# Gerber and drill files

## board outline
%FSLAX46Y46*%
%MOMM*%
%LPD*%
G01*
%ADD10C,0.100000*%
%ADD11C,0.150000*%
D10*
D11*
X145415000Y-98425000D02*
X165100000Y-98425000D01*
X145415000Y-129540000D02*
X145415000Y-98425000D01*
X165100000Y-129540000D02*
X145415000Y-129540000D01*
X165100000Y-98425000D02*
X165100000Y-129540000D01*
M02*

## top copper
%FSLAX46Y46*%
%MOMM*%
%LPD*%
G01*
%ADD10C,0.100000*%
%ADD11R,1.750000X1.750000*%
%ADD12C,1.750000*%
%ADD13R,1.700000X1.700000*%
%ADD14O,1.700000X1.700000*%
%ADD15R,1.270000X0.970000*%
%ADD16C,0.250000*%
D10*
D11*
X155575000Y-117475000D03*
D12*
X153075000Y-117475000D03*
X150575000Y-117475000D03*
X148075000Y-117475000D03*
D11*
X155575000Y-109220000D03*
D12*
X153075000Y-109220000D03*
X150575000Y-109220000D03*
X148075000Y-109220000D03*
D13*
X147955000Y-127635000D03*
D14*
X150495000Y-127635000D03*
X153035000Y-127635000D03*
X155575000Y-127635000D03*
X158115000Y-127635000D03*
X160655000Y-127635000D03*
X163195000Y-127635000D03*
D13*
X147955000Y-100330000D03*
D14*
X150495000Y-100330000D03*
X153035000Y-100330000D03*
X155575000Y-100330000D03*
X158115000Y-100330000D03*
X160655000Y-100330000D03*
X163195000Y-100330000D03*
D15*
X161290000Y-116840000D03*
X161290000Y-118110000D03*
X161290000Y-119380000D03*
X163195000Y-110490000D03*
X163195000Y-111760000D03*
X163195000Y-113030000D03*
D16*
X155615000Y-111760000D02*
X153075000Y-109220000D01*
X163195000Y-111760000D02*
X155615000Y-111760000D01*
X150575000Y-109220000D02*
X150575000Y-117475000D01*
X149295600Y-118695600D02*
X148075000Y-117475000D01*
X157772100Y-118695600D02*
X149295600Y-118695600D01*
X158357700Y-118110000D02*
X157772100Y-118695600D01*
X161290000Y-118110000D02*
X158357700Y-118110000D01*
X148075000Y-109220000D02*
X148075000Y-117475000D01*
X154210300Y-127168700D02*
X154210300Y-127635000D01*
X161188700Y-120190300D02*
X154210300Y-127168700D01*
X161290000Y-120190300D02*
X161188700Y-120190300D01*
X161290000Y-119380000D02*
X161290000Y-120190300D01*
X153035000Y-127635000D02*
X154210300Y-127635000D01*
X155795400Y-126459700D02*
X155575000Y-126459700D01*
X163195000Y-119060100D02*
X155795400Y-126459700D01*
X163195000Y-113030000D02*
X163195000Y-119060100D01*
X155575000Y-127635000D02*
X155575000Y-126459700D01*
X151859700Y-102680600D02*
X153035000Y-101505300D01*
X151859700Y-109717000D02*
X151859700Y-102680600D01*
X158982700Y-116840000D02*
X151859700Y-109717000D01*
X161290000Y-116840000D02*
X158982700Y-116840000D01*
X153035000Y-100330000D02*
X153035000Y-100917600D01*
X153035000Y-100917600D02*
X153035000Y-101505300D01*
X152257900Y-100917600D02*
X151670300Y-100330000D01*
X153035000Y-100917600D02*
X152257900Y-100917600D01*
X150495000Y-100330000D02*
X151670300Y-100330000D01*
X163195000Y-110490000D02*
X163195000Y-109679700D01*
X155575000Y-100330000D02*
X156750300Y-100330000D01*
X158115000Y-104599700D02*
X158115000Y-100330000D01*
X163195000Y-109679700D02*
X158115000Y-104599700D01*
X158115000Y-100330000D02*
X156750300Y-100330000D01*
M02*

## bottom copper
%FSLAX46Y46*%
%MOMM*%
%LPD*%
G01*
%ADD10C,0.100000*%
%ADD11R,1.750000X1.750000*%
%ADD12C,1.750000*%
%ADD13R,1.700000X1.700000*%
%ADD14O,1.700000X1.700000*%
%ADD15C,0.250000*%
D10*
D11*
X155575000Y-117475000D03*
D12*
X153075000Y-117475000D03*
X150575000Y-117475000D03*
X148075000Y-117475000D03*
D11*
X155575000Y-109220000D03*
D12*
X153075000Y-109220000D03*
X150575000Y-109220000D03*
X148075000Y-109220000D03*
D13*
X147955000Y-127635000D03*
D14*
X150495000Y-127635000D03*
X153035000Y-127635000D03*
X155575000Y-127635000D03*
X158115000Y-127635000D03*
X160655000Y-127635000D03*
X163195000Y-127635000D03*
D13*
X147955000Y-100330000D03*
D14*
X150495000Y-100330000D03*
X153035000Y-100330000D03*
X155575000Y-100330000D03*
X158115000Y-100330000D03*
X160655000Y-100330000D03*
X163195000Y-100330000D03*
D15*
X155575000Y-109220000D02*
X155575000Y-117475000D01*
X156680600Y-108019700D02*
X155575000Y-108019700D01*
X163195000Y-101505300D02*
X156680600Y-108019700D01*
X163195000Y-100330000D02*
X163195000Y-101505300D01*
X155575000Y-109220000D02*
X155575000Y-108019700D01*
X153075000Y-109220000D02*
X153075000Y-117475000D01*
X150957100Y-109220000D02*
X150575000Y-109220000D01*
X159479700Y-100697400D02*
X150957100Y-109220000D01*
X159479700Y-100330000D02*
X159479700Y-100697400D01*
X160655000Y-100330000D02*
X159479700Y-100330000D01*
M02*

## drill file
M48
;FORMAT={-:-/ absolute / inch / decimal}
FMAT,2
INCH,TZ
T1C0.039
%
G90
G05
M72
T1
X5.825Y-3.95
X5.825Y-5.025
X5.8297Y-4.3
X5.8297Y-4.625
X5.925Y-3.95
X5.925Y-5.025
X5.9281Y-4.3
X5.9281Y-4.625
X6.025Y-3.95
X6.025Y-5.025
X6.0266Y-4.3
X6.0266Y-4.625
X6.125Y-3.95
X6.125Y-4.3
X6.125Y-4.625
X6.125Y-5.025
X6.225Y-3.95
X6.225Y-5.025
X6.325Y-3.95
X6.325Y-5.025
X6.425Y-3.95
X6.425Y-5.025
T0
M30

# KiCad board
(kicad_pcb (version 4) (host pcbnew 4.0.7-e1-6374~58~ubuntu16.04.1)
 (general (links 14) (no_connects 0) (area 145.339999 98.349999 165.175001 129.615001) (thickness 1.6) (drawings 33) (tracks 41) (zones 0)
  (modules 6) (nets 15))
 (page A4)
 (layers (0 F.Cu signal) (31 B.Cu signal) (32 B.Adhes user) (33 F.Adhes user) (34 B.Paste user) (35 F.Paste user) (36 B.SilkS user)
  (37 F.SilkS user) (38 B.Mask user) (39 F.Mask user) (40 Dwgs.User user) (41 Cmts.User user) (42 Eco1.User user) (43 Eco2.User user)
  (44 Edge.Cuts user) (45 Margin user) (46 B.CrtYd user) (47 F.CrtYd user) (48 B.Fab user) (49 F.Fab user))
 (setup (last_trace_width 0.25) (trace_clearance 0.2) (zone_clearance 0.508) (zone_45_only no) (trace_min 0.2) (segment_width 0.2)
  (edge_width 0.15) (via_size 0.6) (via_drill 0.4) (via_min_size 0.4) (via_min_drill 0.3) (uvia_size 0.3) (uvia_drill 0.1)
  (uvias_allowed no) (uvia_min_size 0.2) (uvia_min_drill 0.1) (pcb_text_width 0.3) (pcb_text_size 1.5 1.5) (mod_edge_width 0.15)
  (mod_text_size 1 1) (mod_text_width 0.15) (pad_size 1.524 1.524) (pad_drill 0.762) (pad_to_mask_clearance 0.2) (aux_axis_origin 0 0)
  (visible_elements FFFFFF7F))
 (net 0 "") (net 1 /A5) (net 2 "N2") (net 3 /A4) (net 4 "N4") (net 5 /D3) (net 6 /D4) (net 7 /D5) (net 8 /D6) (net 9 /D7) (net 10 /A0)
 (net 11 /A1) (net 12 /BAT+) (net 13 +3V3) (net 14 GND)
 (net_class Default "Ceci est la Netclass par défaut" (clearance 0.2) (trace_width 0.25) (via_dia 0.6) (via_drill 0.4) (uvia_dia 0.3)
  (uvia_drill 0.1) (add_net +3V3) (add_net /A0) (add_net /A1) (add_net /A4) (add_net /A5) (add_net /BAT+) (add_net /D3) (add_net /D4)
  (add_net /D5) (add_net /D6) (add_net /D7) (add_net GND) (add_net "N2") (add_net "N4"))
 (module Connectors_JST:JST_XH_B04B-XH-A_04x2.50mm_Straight (layer F.Cu) (at 155.575 117.475 180)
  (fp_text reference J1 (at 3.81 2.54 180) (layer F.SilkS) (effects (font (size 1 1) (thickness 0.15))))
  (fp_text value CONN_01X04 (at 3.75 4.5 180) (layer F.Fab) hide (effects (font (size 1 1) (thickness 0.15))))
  (pad 1 thru_hole rect (at 0 0 180) (size 1.75 1.75) (drill 1) (layers *.Cu *.Mask) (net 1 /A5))
  (pad 2 thru_hole circle (at 2.5 0 180) (size 1.75 1.75) (drill 1) (layers *.Cu *.Mask) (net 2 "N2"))
  (pad 3 thru_hole circle (at 5 0 180) (size 1.75 1.75) (drill 1) (layers *.Cu *.Mask) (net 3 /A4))
  (pad 4 thru_hole circle (at 7.5 0 180) (size 1.75 1.75) (drill 1) (layers *.Cu *.Mask) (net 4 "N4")))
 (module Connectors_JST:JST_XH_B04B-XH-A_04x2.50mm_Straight (layer F.Cu) (at 155.575 109.22 180)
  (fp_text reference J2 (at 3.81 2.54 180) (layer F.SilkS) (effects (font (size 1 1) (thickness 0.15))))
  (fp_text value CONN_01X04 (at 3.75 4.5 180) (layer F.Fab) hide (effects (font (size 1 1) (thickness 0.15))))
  (pad 1 thru_hole rect (at 0 0 180) (size 1.75 1.75) (drill 1) (layers *.Cu *.Mask) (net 1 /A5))
  (pad 2 thru_hole circle (at 2.5 0 180) (size 1.75 1.75) (drill 1) (layers *.Cu *.Mask) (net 2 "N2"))
  (pad 3 thru_hole circle (at 5 0 180) (size 1.75 1.75) (drill 1) (layers *.Cu *.Mask) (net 3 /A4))
  (pad 4 thru_hole circle (at 7.5 0 180) (size 1.75 1.75) (drill 1) (layers *.Cu *.Mask) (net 4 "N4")))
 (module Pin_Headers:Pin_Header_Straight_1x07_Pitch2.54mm (layer B.Cu) (at 147.955 127.635 270)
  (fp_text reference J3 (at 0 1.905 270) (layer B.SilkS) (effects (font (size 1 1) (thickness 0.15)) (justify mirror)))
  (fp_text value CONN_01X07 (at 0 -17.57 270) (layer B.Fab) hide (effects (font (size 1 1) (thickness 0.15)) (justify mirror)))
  (pad 1 thru_hole rect (at 0 0 270) (size 1.7 1.7) (drill 1) (layers *.Cu *.Mask) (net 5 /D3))
  (pad 2 thru_hole oval (at 0 -2.54 270) (size 1.7 1.7) (drill 1) (layers *.Cu *.Mask) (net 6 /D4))
  (pad 3 thru_hole oval (at 0 -5.08 270) (size 1.7 1.7) (drill 1) (layers *.Cu *.Mask) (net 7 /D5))
  (pad 4 thru_hole oval (at 0 -7.62 270) (size 1.7 1.7) (drill 1) (layers *.Cu *.Mask) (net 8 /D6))
  (pad 5 thru_hole oval (at 0 -10.16 270) (size 1.7 1.7) (drill 1) (layers *.Cu *.Mask) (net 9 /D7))
  (pad 6 thru_hole oval (at 0 -12.7 270) (size 1.7 1.7) (drill 1) (layers *.Cu *.Mask) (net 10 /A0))
  (pad 7 thru_hole oval (at 0 -15.24 270) (size 1.7 1.7) (drill 1) (layers *.Cu *.Mask) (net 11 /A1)))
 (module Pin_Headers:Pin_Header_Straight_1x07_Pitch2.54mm (layer B.Cu) (at 147.955 100.33 270)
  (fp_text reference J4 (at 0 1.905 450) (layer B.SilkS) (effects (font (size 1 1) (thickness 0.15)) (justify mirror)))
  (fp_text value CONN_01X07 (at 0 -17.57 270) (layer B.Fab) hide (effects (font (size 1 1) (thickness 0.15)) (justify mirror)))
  (pad 1 thru_hole rect (at 0 0 270) (size 1.7 1.7) (drill 1) (layers *.Cu *.Mask) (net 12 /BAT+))
  (pad 2 thru_hole oval (at 0 -2.54 270) (size 1.7 1.7) (drill 1) (layers *.Cu *.Mask) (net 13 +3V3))
  (pad 3 thru_hole oval (at 0 -5.08 270) (size 1.7 1.7) (drill 1) (layers *.Cu *.Mask) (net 13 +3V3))
  (pad 4 thru_hole oval (at 0 -7.62 270) (size 1.7 1.7) (drill 1) (layers *.Cu *.Mask) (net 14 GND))
  (pad 5 thru_hole oval (at 0 -10.16 270) (size 1.7 1.7) (drill 1) (layers *.Cu *.Mask) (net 14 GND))
  (pad 6 thru_hole oval (at 0 -12.7 270) (size 1.7 1.7) (drill 1) (layers *.Cu *.Mask) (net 3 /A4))
  (pad 7 thru_hole oval (at 0 -15.24 270) (size 1.7 1.7) (drill 1) (layers *.Cu *.Mask) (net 1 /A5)))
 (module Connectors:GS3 (layer F.Cu) (at 161.29 118.11)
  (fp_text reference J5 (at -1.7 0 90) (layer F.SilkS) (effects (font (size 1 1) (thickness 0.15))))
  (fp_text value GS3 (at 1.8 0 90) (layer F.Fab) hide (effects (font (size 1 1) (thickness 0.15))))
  (pad 1 smd rect (at 0 -1.27) (size 1.27 0.97) (layers F.Cu F.Paste F.Mask) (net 13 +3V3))
  (pad 2 smd rect (at 0 0) (size 1.27 0.97) (layers F.Cu F.Paste F.Mask) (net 4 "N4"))
  (pad 3 smd rect (at 0 1.27) (size 1.27 0.97) (layers F.Cu F.Paste F.Mask) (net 7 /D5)))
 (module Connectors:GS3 (layer F.Cu) (at 163.195 111.76)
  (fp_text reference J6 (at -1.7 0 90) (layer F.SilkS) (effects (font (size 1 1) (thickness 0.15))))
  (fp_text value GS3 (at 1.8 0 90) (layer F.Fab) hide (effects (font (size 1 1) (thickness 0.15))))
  (pad 1 smd rect (at 0 -1.27) (size 1.27 0.97) (layers F.Cu F.Paste F.Mask) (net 14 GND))
  (pad 2 smd rect (at 0 0) (size 1.27 0.97) (layers F.Cu F.Paste F.Mask) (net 2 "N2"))
  (pad 3 smd rect (at 0 1.27) (size 1.27 0.97) (layers F.Cu F.Paste F.Mask) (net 8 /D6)))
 (gr_line (start 145.415 98.425) (end 165.1 98.425) (angle 90) (layer Edge.Cuts) (width 0.15))
 (gr_line (start 145.415 129.54) (end 145.415 98.425) (angle 90) (layer Edge.Cuts) (width 0.15))
 (gr_line (start 165.1 129.54) (end 145.415 129.54) (angle 90) (layer Edge.Cuts) (width 0.15))
 (gr_line (start 165.1 98.425) (end 165.1 129.54) (angle 90) (layer Edge.Cuts) (width 0.15))
 (segment (start 155.575 109.22) (end 155.575 117.475) (width 0.25) (layer B.Cu) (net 1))
 (segment (start 156.6806 108.0197) (end 155.575 108.0197) (width 0.25) (layer B.Cu) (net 1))
 (segment (start 163.195 101.5053) (end 156.6806 108.0197) (width 0.25) (layer B.Cu) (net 1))
 (segment (start 163.195 100.33) (end 163.195 101.5053) (width 0.25) (layer B.Cu) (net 1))
 (segment (start 155.575 109.22) (end 155.575 108.0197) (width 0.25) (layer B.Cu) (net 1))
 (segment (start 155.615 111.76) (end 153.075 109.22) (width 0.25) (layer F.Cu) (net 2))
 (segment (start 163.195 111.76) (end 155.615 111.76) (width 0.25) (layer F.Cu) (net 2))
 (segment (start 153.075 109.22) (end 153.075 117.475) (width 0.25) (layer B.Cu) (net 2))
 (segment (start 150.9571 109.22) (end 150.575 109.22) (width 0.25) (layer B.Cu) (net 3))
 (segment (start 159.4797 100.6974) (end 150.9571 109.22) (width 0.25) (layer B.Cu) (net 3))
 (segment (start 159.4797 100.33) (end 159.4797 100.6974) (width 0.25) (layer B.Cu) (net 3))
 (segment (start 160.655 100.33) (end 159.4797 100.33) (width 0.25) (layer B.Cu) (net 3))
 (segment (start 150.575 109.22) (end 150.575 117.475) (width 0.25) (layer F.Cu) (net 3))
 (segment (start 149.2956 118.6956) (end 148.075 117.475) (width 0.25) (layer F.Cu) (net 4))
 (segment (start 157.7721 118.6956) (end 149.2956 118.6956) (width 0.25) (layer F.Cu) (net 4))
 (segment (start 158.3577 118.11) (end 157.7721 118.6956) (width 0.25) (layer F.Cu) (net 4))
 (segment (start 161.29 118.11) (end 158.3577 118.11) (width 0.25) (layer F.Cu) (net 4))
 (segment (start 148.075 109.22) (end 148.075 117.475) (width 0.25) (layer F.Cu) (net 4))
 (segment (start 154.2103 127.1687) (end 154.2103 127.635) (width 0.25) (layer F.Cu) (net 7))
 (segment (start 161.1887 120.1903) (end 154.2103 127.1687) (width 0.25) (layer F.Cu) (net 7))
 (segment (start 161.29 120.1903) (end 161.1887 120.1903) (width 0.25) (layer F.Cu) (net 7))
 (segment (start 161.29 119.38) (end 161.29 120.1903) (width 0.25) (layer F.Cu) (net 7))
 (segment (start 153.035 127.635) (end 154.2103 127.635) (width 0.25) (layer F.Cu) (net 7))
 (segment (start 155.7954 126.4597) (end 155.575 126.4597) (width 0.25) (layer F.Cu) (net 8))
 (segment (start 163.195 119.0601) (end 155.7954 126.4597) (width 0.25) (layer F.Cu) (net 8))
 (segment (start 163.195 113.03) (end 163.195 119.0601) (width 0.25) (layer F.Cu) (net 8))
 (segment (start 155.575 127.635) (end 155.575 126.4597) (width 0.25) (layer F.Cu) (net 8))
 (segment (start 151.8597 102.6806) (end 153.035 101.5053) (width 0.25) (layer F.Cu) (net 13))
 (segment (start 151.8597 109.717) (end 151.8597 102.6806) (width 0.25) (layer F.Cu) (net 13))
 (segment (start 158.9827 116.84) (end 151.8597 109.717) (width 0.25) (layer F.Cu) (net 13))
 (segment (start 161.29 116.84) (end 158.9827 116.84) (width 0.25) (layer F.Cu) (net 13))
 (segment (start 153.035 100.33) (end 153.035 100.9176) (width 0.25) (layer F.Cu) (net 13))
 (segment (start 153.035 100.9176) (end 153.035 101.5053) (width 0.25) (layer F.Cu) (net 13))
 (segment (start 152.2579 100.9176) (end 151.6703 100.33) (width 0.25) (layer F.Cu) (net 13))
 (segment (start 153.035 100.9176) (end 152.2579 100.9176) (width 0.25) (layer F.Cu) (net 13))
 (segment (start 150.495 100.33) (end 151.6703 100.33) (width 0.25) (layer F.Cu) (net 13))
 (segment (start 163.195 110.49) (end 163.195 109.6797) (width 0.25) (layer F.Cu) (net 14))
 (segment (start 155.575 100.33) (end 156.7503 100.33) (width 0.25) (layer F.Cu) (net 14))
 (segment (start 158.115 104.5997) (end 158.115 100.33) (width 0.25) (layer F.Cu) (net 14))
 (segment (start 163.195 109.6797) (end 158.115 104.5997) (width 0.25) (layer F.Cu) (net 14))
 (segment (start 158.115 100.33) (end 156.7503 100.33) (width 0.25) (layer F.Cu) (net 14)))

